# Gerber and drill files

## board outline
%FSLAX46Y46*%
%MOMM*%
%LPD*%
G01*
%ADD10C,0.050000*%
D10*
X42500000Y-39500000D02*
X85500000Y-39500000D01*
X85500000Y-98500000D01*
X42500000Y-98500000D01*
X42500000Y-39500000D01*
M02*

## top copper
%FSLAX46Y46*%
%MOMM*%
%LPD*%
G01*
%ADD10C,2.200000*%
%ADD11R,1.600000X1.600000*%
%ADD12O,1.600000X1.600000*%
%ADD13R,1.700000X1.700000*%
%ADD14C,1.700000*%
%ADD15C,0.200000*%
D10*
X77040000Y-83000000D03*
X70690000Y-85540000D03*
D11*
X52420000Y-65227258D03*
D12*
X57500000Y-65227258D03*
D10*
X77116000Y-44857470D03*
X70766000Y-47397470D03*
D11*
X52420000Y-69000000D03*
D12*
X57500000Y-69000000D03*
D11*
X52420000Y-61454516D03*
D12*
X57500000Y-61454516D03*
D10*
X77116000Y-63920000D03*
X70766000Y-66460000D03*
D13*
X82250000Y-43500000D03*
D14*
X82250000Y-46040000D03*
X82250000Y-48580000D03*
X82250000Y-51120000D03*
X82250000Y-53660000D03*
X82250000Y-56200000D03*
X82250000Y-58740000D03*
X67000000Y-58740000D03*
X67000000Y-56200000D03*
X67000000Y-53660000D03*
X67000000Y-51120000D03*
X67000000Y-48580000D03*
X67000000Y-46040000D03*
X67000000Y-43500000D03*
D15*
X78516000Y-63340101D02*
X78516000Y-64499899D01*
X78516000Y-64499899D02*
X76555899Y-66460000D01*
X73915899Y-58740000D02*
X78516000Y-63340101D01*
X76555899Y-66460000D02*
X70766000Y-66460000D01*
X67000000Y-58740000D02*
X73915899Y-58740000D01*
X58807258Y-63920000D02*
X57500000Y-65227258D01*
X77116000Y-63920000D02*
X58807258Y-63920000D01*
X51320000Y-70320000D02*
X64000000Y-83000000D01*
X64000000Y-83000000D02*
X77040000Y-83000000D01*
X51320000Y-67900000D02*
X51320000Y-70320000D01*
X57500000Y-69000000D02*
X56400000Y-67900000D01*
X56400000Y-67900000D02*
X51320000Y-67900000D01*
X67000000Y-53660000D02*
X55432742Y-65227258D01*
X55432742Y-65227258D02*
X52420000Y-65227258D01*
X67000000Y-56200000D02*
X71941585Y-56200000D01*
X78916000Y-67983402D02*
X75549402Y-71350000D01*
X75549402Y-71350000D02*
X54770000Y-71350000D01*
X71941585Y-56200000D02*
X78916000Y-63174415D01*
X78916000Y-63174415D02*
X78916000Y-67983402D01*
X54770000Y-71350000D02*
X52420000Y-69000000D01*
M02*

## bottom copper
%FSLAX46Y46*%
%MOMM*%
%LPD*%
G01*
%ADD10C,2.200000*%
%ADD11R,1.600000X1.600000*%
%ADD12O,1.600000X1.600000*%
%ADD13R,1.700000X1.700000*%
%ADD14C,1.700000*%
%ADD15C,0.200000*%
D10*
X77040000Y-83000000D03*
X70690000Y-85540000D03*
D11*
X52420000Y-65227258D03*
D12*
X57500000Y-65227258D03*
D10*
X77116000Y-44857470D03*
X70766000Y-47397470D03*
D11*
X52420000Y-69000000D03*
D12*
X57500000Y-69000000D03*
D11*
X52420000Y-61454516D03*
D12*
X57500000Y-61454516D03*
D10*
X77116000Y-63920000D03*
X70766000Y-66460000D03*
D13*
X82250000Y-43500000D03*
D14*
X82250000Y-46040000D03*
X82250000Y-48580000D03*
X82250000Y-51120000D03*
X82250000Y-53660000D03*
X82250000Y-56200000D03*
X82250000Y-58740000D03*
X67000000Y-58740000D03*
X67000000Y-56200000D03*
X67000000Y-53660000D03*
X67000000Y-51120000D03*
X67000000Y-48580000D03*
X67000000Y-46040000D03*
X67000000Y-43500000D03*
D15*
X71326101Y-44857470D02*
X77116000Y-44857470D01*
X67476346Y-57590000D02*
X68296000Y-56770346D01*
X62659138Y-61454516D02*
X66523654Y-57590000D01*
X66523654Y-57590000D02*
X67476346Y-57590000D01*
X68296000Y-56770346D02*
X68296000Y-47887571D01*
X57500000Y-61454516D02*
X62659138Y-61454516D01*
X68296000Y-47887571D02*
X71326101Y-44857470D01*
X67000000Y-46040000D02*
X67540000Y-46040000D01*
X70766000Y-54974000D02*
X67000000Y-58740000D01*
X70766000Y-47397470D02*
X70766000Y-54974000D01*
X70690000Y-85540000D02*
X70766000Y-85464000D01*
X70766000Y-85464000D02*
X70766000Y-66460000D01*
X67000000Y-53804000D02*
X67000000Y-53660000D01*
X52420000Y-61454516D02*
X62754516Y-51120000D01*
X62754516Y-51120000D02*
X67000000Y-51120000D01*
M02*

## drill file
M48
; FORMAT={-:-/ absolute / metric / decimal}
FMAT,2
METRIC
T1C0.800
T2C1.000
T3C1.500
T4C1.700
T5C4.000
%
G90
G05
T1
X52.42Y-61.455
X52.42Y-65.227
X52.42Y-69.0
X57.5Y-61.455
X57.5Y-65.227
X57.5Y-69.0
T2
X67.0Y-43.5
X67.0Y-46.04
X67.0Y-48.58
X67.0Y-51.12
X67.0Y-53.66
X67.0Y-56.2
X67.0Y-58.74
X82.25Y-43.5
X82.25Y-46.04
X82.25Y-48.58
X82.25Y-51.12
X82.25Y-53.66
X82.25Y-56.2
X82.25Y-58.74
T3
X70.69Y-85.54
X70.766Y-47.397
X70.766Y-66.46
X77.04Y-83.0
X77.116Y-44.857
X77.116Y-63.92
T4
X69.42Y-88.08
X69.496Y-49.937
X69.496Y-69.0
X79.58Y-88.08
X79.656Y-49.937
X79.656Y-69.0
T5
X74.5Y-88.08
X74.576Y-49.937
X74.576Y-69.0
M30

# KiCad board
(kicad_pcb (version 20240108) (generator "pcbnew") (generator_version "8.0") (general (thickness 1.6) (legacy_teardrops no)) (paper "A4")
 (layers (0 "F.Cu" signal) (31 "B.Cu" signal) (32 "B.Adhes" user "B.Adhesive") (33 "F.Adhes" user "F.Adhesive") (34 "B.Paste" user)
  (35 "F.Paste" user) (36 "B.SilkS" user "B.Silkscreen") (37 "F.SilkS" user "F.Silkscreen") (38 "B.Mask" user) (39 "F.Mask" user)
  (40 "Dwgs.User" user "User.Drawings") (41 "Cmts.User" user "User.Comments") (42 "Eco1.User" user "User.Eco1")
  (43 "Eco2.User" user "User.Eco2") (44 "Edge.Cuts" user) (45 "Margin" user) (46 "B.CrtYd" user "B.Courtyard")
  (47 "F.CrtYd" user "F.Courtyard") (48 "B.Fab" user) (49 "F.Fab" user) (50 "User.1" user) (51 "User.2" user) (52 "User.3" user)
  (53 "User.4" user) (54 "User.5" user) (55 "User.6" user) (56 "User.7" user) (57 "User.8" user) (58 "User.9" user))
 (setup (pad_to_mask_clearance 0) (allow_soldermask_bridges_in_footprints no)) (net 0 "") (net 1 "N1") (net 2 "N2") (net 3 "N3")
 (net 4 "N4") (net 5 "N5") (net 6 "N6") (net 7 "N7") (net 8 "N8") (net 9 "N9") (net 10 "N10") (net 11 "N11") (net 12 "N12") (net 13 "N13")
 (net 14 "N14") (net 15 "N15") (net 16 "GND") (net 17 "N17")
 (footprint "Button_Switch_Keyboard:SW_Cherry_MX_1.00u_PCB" (layer "F.Cu") (at 77.04 83)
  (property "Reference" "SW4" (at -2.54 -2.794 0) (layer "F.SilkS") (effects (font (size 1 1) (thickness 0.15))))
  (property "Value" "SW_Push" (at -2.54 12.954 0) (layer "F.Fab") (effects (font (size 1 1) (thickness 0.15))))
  (pad "" np_thru_hole circle (at -7.62 5.08) (size 1.7 1.7) (drill 1.7) (layers "*.Cu" "*.Mask"))
  (pad "" np_thru_hole circle (at -2.54 5.08) (size 4 4) (drill 4) (layers "*.Cu" "*.Mask"))
  (pad "" np_thru_hole circle (at 2.54 5.08) (size 1.7 1.7) (drill 1.7) (layers "*.Cu" "*.Mask"))
  (pad "1" thru_hole circle (at 0 0) (size 2.2 2.2) (drill 1.5) (layers "*.Cu" "*.Mask") (remove_unused_layers no) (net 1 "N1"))
  (pad "2" thru_hole circle (at -6.35 2.54) (size 2.2 2.2) (drill 1.5) (layers "*.Cu" "*.Mask") (remove_unused_layers no) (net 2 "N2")))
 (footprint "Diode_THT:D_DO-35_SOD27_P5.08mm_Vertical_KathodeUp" (layer "F.Cu") (at 52.42 65.227258)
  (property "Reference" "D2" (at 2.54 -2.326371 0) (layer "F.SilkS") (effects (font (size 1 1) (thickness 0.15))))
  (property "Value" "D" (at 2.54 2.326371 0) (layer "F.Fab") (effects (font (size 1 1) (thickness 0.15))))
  (pad "1" thru_hole rect (at 0 0) (size 1.6 1.6) (drill 0.8) (layers "*.Cu" "*.Mask") (remove_unused_layers no) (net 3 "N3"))
  (pad "2" thru_hole oval (at 5.08 0) (size 1.6 1.6) (drill 0.8) (layers "*.Cu" "*.Mask") (remove_unused_layers no) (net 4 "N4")))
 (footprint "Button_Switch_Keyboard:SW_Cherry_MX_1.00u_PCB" (layer "F.Cu") (at 77.116 44.85747)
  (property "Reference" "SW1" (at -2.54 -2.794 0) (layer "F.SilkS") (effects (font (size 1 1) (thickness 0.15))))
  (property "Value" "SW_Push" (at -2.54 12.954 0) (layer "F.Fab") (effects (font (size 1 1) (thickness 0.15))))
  (pad "" np_thru_hole circle (at -7.62 5.08) (size 1.7 1.7) (drill 1.7) (layers "*.Cu" "*.Mask"))
  (pad "" np_thru_hole circle (at -2.54 5.08) (size 4 4) (drill 4) (layers "*.Cu" "*.Mask"))
  (pad "" np_thru_hole circle (at 2.54 5.08) (size 1.7 1.7) (drill 1.7) (layers "*.Cu" "*.Mask"))
  (pad "1" thru_hole circle (at 0 0) (size 2.2 2.2) (drill 1.5) (layers "*.Cu" "*.Mask") (remove_unused_layers no) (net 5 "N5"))
  (pad "2" thru_hole circle (at -6.35 2.54) (size 2.2 2.2) (drill 1.5) (layers "*.Cu" "*.Mask") (remove_unused_layers no) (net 2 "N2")))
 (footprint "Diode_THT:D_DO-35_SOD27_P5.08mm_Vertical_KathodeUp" (layer "F.Cu") (at 52.42 69)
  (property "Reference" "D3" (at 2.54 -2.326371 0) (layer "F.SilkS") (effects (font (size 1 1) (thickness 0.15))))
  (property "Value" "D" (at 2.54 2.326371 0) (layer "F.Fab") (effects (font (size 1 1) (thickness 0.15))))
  (pad "1" thru_hole rect (at 0 0) (size 1.6 1.6) (drill 0.8) (layers "*.Cu" "*.Mask") (remove_unused_layers no) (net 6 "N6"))
  (pad "2" thru_hole oval (at 5.08 0) (size 1.6 1.6) (drill 0.8) (layers "*.Cu" "*.Mask") (remove_unused_layers no) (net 1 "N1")))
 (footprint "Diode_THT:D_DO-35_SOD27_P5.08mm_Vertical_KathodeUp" (layer "F.Cu") (at 52.42 61.454516)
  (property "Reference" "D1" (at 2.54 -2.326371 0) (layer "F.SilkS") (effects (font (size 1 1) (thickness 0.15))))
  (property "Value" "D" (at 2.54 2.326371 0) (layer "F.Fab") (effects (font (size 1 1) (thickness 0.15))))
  (pad "1" thru_hole rect (at 0 0) (size 1.6 1.6) (drill 0.8) (layers "*.Cu" "*.Mask") (remove_unused_layers no) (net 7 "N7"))
  (pad "2" thru_hole oval (at 5.08 0) (size 1.6 1.6) (drill 0.8) (layers "*.Cu" "*.Mask") (remove_unused_layers no) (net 5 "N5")))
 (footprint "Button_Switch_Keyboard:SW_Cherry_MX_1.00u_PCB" (layer "F.Cu") (at 77.116 63.92)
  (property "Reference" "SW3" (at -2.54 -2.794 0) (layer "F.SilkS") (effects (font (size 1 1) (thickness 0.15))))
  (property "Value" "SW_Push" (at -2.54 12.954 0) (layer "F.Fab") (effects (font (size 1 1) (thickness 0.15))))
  (pad "" np_thru_hole circle (at -7.62 5.08) (size 1.7 1.7) (drill 1.7) (layers "*.Cu" "*.Mask"))
  (pad "" np_thru_hole circle (at -2.54 5.08) (size 4 4) (drill 4) (layers "*.Cu" "*.Mask"))
  (pad "" np_thru_hole circle (at 2.54 5.08) (size 1.7 1.7) (drill 1.7) (layers "*.Cu" "*.Mask"))
  (pad "1" thru_hole circle (at 0 0) (size 2.2 2.2) (drill 1.5) (layers "*.Cu" "*.Mask") (remove_unused_layers no) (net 4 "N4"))
  (pad "2" thru_hole circle (at -6.35 2.54) (size 2.2 2.2) (drill 1.5) (layers "*.Cu" "*.Mask") (remove_unused_layers no) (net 2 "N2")))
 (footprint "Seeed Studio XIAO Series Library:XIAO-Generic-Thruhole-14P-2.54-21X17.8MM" (layer "B.Cu") (at 74.625 51.12 180)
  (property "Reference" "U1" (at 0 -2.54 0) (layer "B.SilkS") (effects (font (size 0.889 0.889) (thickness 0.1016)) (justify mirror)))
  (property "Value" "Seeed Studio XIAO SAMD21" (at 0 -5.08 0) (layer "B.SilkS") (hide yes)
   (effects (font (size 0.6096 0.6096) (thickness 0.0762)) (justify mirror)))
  (pad "1" thru_hole rect (at -7.625 7.62 180) (size 1.7 1.7) (drill 1) (layers "*.Cu" "*.Mask") (remove_unused_layers no) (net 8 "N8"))
  (pad "2" thru_hole circle (at -7.625 5.08 180) (size 1.7 1.7) (drill 1) (layers "*.Cu" "*.Mask") (remove_unused_layers no) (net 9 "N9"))
  (pad "3" thru_hole circle (at -7.625 2.54 180) (size 1.7 1.7) (drill 1) (layers "*.Cu" "*.Mask") (remove_unused_layers no) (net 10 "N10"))
  (pad "4" thru_hole circle (at -7.625 0 180) (size 1.7 1.7) (drill 1) (layers "*.Cu" "*.Mask") (remove_unused_layers no) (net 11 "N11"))
  (pad "5" thru_hole circle (at -7.625 -2.54 180) (size 1.7 1.7) (drill 1) (layers "*.Cu" "*.Mask") (remove_unused_layers no) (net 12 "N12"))
  (pad "6" thru_hole circle (at -7.625 -5.08) (size 1.7 1.7) (drill 1) (layers "*.Cu" "*.Mask") (remove_unused_layers no) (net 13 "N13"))
  (pad "7" thru_hole circle (at -7.625 -7.62 180) (size 1.7 1.7) (drill 1) (layers "*.Cu" "*.Mask") (remove_unused_layers no) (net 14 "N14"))
  (pad "8" thru_hole circle (at 7.625 -7.62 180) (size 1.7 1.7) (drill 1) (layers "*.Cu" "*.Mask") (remove_unused_layers no) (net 2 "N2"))
  (pad "9" thru_hole circle (at 7.625 -5.08 180) (size 1.7 1.7) (drill 1) (layers "*.Cu" "*.Mask") (remove_unused_layers no) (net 6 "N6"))
  (pad "10" thru_hole circle (at 7.625 -2.54 180) (size 1.7 1.7) (drill 1) (layers "*.Cu" "*.Mask") (remove_unused_layers no) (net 3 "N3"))
  (pad "11" thru_hole circle (at 7.625 0 180) (size 1.7 1.7) (drill 1) (layers "*.Cu" "*.Mask") (remove_unused_layers no) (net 7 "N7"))
  (pad "12" thru_hole circle (at 7.625 2.54 180) (size 1.7 1.7) (drill 1) (layers "*.Cu" "*.Mask") (remove_unused_layers no) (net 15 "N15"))
  (pad "13" thru_hole circle (at 7.625 5.08 180) (size 1.7 1.7) (drill 1) (layers "*.Cu" "*.Mask") (remove_unused_layers no) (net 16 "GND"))
  (pad "14" thru_hole circle (at 7.625 7.62 180) (size 1.7 1.7) (drill 1) (layers "*.Cu" "*.Mask") (remove_unused_layers no) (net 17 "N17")))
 (gr_rect (start 42.5 39.5) (end 85.5 98.5) (stroke (width 0.05) (type default)) (fill none) (layer "Edge.Cuts"))
 (segment (start 71.326101 44.85747) (end 77.116 44.85747) (width 0.2) (layer "B.Cu") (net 5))
 (segment (start 67.476346 57.59) (end 68.296 56.770346) (width 0.2) (layer "B.Cu") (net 5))
 (segment (start 62.659138 61.454516) (end 66.523654 57.59) (width 0.2) (layer "B.Cu") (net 5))
 (segment (start 66.523654 57.59) (end 67.476346 57.59) (width 0.2) (layer "B.Cu") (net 5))
 (segment (start 68.296 56.770346) (end 68.296 47.887571) (width 0.2) (layer "B.Cu") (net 5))
 (segment (start 57.5 61.454516) (end 62.659138 61.454516) (width 0.2) (layer "B.Cu") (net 5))
 (segment (start 68.296 47.887571) (end 71.326101 44.85747) (width 0.2) (layer "B.Cu") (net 5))
 (segment (start 67 46.04) (end 67.54 46.04) (width 0.2) (layer "B.Cu") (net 16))
 (segment (start 78.516 63.340101) (end 78.516 64.499899) (width 0.2) (layer "F.Cu") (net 2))
 (segment (start 78.516 64.499899) (end 76.555899 66.46) (width 0.2) (layer "F.Cu") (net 2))
 (segment (start 73.915899 58.74) (end 78.516 63.340101) (width 0.2) (layer "F.Cu") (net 2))
 (segment (start 76.555899 66.46) (end 70.766 66.46) (width 0.2) (layer "F.Cu") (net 2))
 (segment (start 67 58.74) (end 73.915899 58.74) (width 0.2) (layer "F.Cu") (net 2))
 (segment (start 70.766 54.974) (end 67 58.74) (width 0.2) (layer "B.Cu") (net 2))
 (segment (start 70.766 47.39747) (end 70.766 54.974) (width 0.2) (layer "B.Cu") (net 2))
 (segment (start 70.69 85.54) (end 70.766 85.464) (width 0.2) (layer "B.Cu") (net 2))
 (segment (start 70.766 85.464) (end 70.766 66.46) (width 0.2) (layer "B.Cu") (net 2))
 (segment (start 58.807258 63.92) (end 57.5 65.227258) (width 0.2) (layer "F.Cu") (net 4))
 (segment (start 77.116 63.92) (end 58.807258 63.92) (width 0.2) (layer "F.Cu") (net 4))
 (segment (start 51.32 70.32) (end 64 83) (width 0.2) (layer "F.Cu") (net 1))
 (segment (start 64 83) (end 77.04 83) (width 0.2) (layer "F.Cu") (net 1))
 (segment (start 51.32 67.9) (end 51.32 70.32) (width 0.2) (layer "F.Cu") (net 1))
 (segment (start 57.5 69) (end 56.4 67.9) (width 0.2) (layer "F.Cu") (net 1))
 (segment (start 56.4 67.9) (end 51.32 67.9) (width 0.2) (layer "F.Cu") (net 1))
 (segment (start 67 53.66) (end 55.432742 65.227258) (width 0.2) (layer "F.Cu") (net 3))
 (segment (start 55.432742 65.227258) (end 52.42 65.227258) (width 0.2) (layer "F.Cu") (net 3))
 (segment (start 67 53.804) (end 67 53.66) (width 0.2) (layer "B.Cu") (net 3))
 (segment (start 52.42 61.454516) (end 62.754516 51.12) (width 0.2) (layer "B.Cu") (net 7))
 (segment (start 62.754516 51.12) (end 67 51.12) (width 0.2) (layer "B.Cu") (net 7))
 (segment (start 67 56.2) (end 71.941585 56.2) (width 0.2) (layer "F.Cu") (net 6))
 (segment (start 78.916 67.983402) (end 75.549402 71.35) (width 0.2) (layer "F.Cu") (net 6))
 (segment (start 75.549402 71.35) (end 54.77 71.35) (width 0.2) (layer "F.Cu") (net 6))
 (segment (start 71.941585 56.2) (end 78.916 63.174415) (width 0.2) (layer "F.Cu") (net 6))
 (segment (start 78.916 63.174415) (end 78.916 67.983402) (width 0.2) (layer "F.Cu") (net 6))
 (segment (start 54.77 71.35) (end 52.42 69) (width 0.2) (layer "F.Cu") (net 6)))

